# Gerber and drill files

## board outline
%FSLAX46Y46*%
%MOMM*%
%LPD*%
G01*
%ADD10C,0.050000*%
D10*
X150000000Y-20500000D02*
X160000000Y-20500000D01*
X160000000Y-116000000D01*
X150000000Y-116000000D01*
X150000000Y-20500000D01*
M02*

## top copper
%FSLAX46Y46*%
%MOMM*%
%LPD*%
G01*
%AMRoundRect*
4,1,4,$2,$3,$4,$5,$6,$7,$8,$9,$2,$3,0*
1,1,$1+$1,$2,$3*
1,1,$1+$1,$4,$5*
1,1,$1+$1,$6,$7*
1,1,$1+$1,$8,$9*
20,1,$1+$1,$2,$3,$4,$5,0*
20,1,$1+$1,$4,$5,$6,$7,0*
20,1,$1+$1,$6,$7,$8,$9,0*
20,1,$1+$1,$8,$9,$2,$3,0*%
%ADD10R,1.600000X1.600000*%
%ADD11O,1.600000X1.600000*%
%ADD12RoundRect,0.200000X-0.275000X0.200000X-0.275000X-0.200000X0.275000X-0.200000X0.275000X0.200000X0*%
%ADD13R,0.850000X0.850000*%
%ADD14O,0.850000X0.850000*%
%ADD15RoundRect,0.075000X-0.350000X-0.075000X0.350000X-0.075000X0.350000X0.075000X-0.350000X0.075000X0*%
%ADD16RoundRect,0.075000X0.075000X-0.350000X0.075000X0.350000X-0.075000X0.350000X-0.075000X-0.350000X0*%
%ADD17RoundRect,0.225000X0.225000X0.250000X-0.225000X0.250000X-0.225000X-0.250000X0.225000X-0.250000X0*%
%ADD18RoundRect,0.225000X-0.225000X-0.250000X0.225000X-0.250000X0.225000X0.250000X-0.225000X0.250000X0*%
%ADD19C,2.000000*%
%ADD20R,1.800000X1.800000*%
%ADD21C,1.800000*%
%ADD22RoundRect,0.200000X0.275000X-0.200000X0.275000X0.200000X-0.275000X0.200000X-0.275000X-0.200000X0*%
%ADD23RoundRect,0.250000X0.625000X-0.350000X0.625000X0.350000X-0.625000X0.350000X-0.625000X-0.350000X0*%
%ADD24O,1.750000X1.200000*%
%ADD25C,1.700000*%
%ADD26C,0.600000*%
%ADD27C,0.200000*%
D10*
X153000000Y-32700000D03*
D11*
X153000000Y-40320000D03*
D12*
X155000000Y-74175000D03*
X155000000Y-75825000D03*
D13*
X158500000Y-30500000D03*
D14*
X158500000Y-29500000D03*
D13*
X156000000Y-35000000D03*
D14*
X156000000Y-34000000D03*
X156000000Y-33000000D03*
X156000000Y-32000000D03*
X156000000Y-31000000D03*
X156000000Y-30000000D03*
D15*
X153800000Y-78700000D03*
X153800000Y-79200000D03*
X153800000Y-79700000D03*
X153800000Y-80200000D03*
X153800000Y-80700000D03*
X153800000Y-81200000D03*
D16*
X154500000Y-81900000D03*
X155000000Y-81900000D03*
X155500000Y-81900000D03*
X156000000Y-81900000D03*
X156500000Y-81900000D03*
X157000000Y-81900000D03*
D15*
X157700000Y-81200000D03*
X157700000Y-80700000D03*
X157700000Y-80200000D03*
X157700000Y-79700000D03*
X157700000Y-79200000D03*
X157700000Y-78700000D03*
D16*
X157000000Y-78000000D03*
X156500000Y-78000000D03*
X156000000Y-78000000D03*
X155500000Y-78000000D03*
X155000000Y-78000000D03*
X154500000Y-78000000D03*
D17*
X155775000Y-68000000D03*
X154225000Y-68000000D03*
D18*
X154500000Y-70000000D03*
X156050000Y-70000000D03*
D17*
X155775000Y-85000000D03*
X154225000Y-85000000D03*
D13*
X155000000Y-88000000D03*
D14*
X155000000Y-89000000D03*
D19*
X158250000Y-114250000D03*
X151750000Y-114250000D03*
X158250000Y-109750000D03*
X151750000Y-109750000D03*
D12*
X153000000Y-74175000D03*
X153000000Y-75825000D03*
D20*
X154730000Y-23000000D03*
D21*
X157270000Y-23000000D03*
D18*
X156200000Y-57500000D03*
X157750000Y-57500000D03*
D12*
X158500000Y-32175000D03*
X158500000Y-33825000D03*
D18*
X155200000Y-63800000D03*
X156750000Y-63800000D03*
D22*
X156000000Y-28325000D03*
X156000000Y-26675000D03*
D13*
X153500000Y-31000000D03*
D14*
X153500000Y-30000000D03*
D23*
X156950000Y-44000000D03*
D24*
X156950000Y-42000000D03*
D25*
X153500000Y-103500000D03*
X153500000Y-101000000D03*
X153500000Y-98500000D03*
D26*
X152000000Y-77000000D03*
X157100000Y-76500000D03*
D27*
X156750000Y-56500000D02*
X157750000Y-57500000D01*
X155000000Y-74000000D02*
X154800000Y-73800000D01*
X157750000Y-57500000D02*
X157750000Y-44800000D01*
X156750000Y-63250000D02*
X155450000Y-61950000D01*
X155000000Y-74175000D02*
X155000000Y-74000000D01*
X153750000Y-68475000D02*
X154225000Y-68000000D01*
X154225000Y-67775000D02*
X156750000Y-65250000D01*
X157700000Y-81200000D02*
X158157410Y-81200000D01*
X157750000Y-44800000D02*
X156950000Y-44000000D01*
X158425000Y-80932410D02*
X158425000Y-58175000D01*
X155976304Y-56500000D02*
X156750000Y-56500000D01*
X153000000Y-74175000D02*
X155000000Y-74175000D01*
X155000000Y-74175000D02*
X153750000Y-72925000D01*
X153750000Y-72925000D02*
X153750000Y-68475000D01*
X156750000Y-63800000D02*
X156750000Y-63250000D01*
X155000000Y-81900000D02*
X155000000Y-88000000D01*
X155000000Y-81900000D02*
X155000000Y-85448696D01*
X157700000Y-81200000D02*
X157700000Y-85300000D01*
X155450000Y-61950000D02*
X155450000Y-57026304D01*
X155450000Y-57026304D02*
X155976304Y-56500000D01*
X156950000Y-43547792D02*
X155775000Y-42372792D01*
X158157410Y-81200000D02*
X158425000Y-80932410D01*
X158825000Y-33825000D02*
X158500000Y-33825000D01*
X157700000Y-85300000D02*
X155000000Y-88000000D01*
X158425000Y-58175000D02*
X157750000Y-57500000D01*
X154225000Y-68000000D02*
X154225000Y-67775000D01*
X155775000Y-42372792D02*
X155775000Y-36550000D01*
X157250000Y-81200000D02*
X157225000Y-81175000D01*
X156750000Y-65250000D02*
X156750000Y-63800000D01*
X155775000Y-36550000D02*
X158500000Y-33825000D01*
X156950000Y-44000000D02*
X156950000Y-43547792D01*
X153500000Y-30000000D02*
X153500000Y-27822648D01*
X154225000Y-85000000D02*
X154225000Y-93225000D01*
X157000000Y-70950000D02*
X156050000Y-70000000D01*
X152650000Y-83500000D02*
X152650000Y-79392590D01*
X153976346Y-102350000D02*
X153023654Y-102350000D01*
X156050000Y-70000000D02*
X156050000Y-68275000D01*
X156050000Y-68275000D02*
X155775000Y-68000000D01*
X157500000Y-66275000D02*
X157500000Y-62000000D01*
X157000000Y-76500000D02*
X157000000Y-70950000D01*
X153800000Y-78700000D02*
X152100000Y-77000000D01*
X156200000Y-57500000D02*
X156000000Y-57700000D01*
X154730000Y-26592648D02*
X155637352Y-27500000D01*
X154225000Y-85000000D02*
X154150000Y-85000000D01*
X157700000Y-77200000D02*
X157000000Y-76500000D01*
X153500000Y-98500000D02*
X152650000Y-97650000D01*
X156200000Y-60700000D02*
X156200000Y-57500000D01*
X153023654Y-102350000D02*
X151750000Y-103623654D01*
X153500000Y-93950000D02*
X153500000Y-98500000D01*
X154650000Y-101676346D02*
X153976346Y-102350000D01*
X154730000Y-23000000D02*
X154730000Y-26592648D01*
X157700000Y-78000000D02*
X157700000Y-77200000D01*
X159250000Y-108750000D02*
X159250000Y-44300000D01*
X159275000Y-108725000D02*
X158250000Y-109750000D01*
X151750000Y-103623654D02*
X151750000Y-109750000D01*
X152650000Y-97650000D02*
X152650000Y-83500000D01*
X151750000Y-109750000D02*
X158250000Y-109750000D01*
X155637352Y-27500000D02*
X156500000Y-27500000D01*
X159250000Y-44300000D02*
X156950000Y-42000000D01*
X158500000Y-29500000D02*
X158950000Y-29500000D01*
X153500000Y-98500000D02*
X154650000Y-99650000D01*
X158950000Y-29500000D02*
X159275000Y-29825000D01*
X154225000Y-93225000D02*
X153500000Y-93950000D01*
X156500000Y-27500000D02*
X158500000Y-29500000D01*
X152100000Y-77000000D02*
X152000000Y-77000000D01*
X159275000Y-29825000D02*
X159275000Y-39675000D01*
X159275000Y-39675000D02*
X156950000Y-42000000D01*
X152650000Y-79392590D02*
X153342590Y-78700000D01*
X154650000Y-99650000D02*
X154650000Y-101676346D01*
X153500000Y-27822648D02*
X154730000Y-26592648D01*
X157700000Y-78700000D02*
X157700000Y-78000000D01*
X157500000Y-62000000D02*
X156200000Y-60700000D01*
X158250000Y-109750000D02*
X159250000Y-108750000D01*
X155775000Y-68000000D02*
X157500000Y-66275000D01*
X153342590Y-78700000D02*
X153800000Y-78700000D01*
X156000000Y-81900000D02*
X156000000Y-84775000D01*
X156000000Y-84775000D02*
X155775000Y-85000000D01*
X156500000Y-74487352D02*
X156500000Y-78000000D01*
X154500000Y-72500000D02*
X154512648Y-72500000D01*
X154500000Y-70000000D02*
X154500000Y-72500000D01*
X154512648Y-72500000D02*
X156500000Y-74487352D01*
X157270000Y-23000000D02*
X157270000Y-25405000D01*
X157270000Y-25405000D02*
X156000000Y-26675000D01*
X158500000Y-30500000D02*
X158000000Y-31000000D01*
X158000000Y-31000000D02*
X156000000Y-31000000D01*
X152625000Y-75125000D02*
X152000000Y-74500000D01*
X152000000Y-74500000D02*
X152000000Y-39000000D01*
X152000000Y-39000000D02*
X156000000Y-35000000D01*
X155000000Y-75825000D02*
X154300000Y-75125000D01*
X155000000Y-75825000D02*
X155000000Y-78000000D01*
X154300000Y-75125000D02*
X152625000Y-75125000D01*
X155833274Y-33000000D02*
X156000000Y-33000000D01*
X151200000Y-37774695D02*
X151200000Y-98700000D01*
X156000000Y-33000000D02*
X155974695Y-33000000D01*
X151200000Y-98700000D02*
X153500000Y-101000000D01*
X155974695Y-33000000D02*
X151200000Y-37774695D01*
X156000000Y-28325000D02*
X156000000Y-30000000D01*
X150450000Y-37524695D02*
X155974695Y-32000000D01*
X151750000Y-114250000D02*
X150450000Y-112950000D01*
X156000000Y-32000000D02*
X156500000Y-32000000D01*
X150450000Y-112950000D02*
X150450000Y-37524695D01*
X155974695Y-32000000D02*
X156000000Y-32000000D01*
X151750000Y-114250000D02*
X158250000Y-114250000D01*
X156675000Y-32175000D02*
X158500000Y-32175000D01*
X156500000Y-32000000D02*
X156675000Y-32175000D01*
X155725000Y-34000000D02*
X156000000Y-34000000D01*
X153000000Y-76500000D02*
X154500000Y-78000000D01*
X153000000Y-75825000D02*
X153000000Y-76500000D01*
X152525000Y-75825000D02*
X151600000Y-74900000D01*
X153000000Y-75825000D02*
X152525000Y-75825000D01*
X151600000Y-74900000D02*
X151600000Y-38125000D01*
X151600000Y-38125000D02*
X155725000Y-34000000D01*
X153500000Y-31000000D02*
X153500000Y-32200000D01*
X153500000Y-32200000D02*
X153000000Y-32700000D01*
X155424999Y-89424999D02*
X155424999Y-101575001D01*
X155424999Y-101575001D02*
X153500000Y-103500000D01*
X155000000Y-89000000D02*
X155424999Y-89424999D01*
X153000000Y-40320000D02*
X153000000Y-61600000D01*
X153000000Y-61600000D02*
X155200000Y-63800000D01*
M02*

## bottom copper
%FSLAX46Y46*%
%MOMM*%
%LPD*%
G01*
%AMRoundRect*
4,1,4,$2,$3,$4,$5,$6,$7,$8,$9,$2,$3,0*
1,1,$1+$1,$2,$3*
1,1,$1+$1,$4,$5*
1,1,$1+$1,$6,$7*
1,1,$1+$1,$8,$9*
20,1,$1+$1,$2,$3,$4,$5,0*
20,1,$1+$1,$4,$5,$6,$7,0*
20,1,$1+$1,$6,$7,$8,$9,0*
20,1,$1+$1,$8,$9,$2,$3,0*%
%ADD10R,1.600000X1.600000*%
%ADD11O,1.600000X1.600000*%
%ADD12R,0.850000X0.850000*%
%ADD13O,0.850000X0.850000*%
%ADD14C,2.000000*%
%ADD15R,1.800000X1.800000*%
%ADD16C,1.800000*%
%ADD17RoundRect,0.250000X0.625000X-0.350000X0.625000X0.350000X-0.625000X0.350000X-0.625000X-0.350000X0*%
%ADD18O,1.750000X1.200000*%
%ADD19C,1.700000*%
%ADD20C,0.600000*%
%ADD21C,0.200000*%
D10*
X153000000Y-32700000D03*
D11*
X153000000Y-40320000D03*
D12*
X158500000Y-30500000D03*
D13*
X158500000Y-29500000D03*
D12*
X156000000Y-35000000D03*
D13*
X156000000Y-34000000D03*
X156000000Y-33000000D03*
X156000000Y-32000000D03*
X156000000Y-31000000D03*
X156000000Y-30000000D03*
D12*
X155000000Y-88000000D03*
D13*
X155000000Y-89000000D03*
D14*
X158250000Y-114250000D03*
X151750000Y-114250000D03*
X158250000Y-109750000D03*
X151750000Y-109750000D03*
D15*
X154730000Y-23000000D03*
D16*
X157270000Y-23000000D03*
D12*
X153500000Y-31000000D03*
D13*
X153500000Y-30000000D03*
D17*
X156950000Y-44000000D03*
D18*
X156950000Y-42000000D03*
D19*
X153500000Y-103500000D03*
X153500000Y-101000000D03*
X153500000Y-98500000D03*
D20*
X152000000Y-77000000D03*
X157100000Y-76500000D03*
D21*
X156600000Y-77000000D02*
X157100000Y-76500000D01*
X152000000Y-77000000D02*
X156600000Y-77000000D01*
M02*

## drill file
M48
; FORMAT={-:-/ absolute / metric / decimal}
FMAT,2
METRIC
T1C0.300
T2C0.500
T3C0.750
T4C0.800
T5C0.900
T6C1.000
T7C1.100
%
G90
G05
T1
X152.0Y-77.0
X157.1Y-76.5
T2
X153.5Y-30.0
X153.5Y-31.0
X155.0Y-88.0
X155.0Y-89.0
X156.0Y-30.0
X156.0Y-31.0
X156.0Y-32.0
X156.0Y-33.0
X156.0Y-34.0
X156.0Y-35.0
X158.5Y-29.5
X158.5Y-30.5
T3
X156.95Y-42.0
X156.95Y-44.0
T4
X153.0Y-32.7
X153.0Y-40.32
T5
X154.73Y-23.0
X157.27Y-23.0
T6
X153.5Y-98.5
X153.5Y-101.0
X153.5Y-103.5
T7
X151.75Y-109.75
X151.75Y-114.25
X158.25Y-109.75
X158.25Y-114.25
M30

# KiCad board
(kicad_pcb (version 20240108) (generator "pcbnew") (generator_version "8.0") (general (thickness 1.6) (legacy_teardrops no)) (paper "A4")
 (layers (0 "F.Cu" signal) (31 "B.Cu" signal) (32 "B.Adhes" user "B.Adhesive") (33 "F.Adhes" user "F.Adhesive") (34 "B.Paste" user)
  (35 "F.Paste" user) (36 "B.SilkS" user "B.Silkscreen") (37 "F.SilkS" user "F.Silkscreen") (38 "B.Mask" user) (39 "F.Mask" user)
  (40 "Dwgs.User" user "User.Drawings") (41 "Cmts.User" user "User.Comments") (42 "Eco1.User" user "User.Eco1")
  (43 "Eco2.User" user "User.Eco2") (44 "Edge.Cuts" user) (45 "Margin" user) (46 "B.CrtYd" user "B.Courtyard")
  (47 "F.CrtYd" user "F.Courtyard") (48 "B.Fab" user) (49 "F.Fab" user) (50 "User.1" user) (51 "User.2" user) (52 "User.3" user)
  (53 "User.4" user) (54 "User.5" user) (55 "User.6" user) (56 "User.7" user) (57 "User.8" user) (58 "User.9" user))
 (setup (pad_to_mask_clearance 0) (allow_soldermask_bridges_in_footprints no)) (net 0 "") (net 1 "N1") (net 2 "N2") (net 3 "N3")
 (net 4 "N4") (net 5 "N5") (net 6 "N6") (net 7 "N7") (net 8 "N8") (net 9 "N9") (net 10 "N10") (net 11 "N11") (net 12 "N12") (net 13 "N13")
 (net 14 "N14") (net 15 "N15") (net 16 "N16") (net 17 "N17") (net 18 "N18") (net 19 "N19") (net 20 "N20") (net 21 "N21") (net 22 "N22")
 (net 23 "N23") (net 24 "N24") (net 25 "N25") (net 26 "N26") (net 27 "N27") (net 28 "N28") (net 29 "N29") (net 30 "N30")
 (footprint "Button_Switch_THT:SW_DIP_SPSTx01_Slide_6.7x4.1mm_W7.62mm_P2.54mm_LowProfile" (layer "F.Cu") (at 153 32.7 -90)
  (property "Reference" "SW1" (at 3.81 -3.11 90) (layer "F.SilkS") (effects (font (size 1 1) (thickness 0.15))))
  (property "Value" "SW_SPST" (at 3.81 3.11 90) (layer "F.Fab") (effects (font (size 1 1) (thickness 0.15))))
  (pad "1" thru_hole rect (at 0 0 270) (size 1.6 1.6) (drill 0.8) (layers "*.Cu" "*.Mask") (remove_unused_layers no) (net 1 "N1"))
  (pad "2" thru_hole oval (at 7.62 0 270) (size 1.6 1.6) (drill 0.8) (layers "*.Cu" "*.Mask") (remove_unused_layers no) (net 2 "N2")))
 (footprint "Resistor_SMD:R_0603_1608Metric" (layer "F.Cu") (at 155 75 -90)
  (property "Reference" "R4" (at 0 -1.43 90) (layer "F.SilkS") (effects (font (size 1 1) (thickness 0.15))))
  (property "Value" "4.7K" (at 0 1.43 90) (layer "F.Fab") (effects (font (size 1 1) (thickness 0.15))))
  (pad "1" smd roundrect (at -0.825 0 270) (size 0.8 0.95) (layers "F.Cu" "F.Paste" "F.Mask") (roundrect_rratio 0.25) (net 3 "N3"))
  (pad "2" smd roundrect (at 0.825 0 270) (size 0.8 0.95) (layers "F.Cu" "F.Paste" "F.Mask") (roundrect_rratio 0.25) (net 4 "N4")))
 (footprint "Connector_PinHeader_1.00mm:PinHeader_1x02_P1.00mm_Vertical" (layer "F.Cu") (at 158.5 30.5 180)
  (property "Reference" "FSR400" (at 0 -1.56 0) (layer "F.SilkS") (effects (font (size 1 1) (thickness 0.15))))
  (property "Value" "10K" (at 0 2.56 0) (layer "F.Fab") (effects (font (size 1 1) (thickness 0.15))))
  (pad "1" thru_hole rect (at 0 0 180) (size 0.85 0.85) (drill 0.5) (layers "*.Cu" "*.Mask") (remove_unused_layers no) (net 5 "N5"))
  (pad "2" thru_hole oval (at 0 1 180) (size 0.85 0.85) (drill 0.5) (layers "*.Cu" "*.Mask") (remove_unused_layers no) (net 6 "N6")))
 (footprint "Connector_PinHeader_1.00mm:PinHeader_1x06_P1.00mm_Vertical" (layer "F.Cu") (at 156 35 180)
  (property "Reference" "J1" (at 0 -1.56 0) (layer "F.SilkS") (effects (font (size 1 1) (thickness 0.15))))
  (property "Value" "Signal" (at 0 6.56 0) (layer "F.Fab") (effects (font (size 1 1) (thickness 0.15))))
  (pad "1" thru_hole rect (at 0 0 180) (size 0.85 0.85) (drill 0.5) (layers "*.Cu" "*.Mask") (remove_unused_layers no) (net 4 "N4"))
  (pad "2" thru_hole oval (at 0 1 180) (size 0.85 0.85) (drill 0.5) (layers "*.Cu" "*.Mask") (remove_unused_layers no) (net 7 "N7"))
  (pad "3" thru_hole oval (at 0 2 180) (size 0.85 0.85) (drill 0.5) (layers "*.Cu" "*.Mask") (remove_unused_layers no) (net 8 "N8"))
  (pad "4" thru_hole oval (at 0 3 180) (size 0.85 0.85) (drill 0.5) (layers "*.Cu" "*.Mask") (remove_unused_layers no) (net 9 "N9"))
  (pad "5" thru_hole oval (at 0 4 180) (size 0.85 0.85) (drill 0.5) (layers "*.Cu" "*.Mask") (remove_unused_layers no) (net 5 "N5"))
  (pad "6" thru_hole oval (at 0 5 180) (size 0.85 0.85) (drill 0.5) (layers "*.Cu" "*.Mask") (remove_unused_layers no) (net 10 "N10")))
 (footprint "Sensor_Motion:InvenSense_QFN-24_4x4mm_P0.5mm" (layer "F.Cu") (at 155.75 79.95)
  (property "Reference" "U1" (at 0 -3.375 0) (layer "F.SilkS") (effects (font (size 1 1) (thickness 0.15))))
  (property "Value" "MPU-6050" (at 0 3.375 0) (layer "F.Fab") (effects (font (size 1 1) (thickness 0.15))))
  (pad "1" smd roundrect (at -1.95 -1.25) (size 0.85 0.3) (layers "F.Cu" "F.Paste" "F.Mask") (roundrect_rratio 0.25) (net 6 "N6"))
  (pad "2" smd roundrect (at -1.95 -0.75) (size 0.85 0.3) (layers "F.Cu" "F.Paste" "F.Mask") (roundrect_rratio 0.25) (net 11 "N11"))
  (pad "3" smd roundrect (at -1.95 -0.25) (size 0.85 0.3) (layers "F.Cu" "F.Paste" "F.Mask") (roundrect_rratio 0.25) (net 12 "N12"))
  (pad "4" smd roundrect (at -1.95 0.25) (size 0.85 0.3) (layers "F.Cu" "F.Paste" "F.Mask") (roundrect_rratio 0.25) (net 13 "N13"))
  (pad "5" smd roundrect (at -1.95 0.75) (size 0.85 0.3) (layers "F.Cu" "F.Paste" "F.Mask") (roundrect_rratio 0.25) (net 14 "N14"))
  (pad "6" smd roundrect (at -1.95 1.25) (size 0.85 0.3) (layers "F.Cu" "F.Paste" "F.Mask") (roundrect_rratio 0.25) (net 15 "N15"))
  (pad "7" smd roundrect (at -1.25 1.95 90) (size 0.85 0.3) (layers "F.Cu" "F.Paste" "F.Mask") (roundrect_rratio 0.25) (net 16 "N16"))
  (pad "8" smd roundrect (at -0.75 1.95 90) (size 0.85 0.3) (layers "F.Cu" "F.Paste" "F.Mask") (roundrect_rratio 0.25) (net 3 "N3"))
  (pad "9" smd roundrect (at -0.25 1.95 90) (size 0.85 0.3) (layers "F.Cu" "F.Paste" "F.Mask") (roundrect_rratio 0.25) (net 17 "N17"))
  (pad "10" smd roundrect (at 0.25 1.95 90) (size 0.85 0.3) (layers "F.Cu" "F.Paste" "F.Mask") (roundrect_rratio 0.25) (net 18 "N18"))
  (pad "11" smd roundrect (at 0.75 1.95 90) (size 0.85 0.3) (layers "F.Cu" "F.Paste" "F.Mask") (roundrect_rratio 0.25) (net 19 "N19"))
  (pad "12" smd roundrect (at 1.25 1.95 90) (size 0.85 0.3) (layers "F.Cu" "F.Paste" "F.Mask") (roundrect_rratio 0.25) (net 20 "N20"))
  (pad "13" smd roundrect (at 1.95 1.25) (size 0.85 0.3) (layers "F.Cu" "F.Paste" "F.Mask") (roundrect_rratio 0.25) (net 3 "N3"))
  (pad "14" smd roundrect (at 1.95 0.75) (size 0.85 0.3) (layers "F.Cu" "F.Paste" "F.Mask") (roundrect_rratio 0.25) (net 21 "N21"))
  (pad "15" smd roundrect (at 1.95 0.25) (size 0.85 0.3) (layers "F.Cu" "F.Paste" "F.Mask") (roundrect_rratio 0.25) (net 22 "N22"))
  (pad "16" smd roundrect (at 1.95 -0.25) (size 0.85 0.3) (layers "F.Cu" "F.Paste" "F.Mask") (roundrect_rratio 0.25) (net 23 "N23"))
  (pad "17" smd roundrect (at 1.95 -0.75) (size 0.85 0.3) (layers "F.Cu" "F.Paste" "F.Mask") (roundrect_rratio 0.25) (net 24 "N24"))
  (pad "18" smd roundrect (at 1.95 -1.25) (size 0.85 0.3) (layers "F.Cu" "F.Paste" "F.Mask") (roundrect_rratio 0.25) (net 6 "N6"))
  (pad "19" smd roundrect (at 1.25 -1.95 90) (size 0.85 0.3) (layers "F.Cu" "F.Paste" "F.Mask") (roundrect_rratio 0.25) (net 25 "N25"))
  (pad "20" smd roundrect (at 0.75 -1.95 90) (size 0.85 0.3) (layers "F.Cu" "F.Paste" "F.Mask") (roundrect_rratio 0.25) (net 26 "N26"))
  (pad "21" smd roundrect (at 0.25 -1.95 90) (size 0.85 0.3) (layers "F.Cu" "F.Paste" "F.Mask") (roundrect_rratio 0.25) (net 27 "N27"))
  (pad "22" smd roundrect (at -0.25 -1.95 90) (size 0.85 0.3) (layers "F.Cu" "F.Paste" "F.Mask") (roundrect_rratio 0.25) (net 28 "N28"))
  (pad "23" smd roundrect (at -0.75 -1.95 90) (size 0.85 0.3) (layers "F.Cu" "F.Paste" "F.Mask") (roundrect_rratio 0.25) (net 4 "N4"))
  (pad "24" smd roundrect (at -1.25 -1.95 90) (size 0.85 0.3) (layers "F.Cu" "F.Paste" "F.Mask") (roundrect_rratio 0.25) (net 7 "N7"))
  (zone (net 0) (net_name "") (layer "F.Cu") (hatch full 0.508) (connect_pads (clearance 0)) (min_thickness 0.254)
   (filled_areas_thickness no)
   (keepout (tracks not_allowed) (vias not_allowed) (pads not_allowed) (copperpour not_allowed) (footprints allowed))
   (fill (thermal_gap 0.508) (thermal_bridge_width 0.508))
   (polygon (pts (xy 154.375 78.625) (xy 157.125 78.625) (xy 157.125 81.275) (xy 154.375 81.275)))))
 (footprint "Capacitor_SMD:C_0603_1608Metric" (layer "F.Cu") (at 155 68 180)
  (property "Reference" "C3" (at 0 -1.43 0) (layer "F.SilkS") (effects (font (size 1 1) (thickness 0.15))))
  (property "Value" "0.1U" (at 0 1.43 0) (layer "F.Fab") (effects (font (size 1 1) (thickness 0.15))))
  (pad "1" smd roundrect (at -0.775 0 180) (size 0.9 0.95) (layers "F.Cu" "F.Paste" "F.Mask") (roundrect_rratio 0.25) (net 6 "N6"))
  (pad "2" smd roundrect (at 0.775 0 180) (size 0.9 0.95) (layers "F.Cu" "F.Paste" "F.Mask") (roundrect_rratio 0.25) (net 3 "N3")))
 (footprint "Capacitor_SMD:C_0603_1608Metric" (layer "F.Cu") (at 155.275 70)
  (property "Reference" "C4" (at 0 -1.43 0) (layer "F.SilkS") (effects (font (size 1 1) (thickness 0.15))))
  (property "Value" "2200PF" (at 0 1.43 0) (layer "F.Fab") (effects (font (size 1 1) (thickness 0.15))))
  (pad "1" smd roundrect (at -0.775 0) (size 0.9 0.95) (layers "F.Cu" "F.Paste" "F.Mask") (roundrect_rratio 0.25) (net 26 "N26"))
  (pad "2" smd roundrect (at 0.775 0) (size 0.9 0.95) (layers "F.Cu" "F.Paste" "F.Mask") (roundrect_rratio 0.25) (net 6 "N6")))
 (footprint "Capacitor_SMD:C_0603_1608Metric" (layer "F.Cu") (at 155 85 180)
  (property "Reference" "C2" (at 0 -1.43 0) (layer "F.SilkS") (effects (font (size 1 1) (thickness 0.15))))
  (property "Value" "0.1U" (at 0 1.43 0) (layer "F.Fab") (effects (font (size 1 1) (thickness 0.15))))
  (pad "1" smd roundrect (at -0.775 0 180) (size 0.9 0.95) (layers "F.Cu" "F.Paste" "F.Mask") (roundrect_rratio 0.25) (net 18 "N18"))
  (pad "2" smd roundrect (at 0.775 0 180) (size 0.9 0.95) (layers "F.Cu" "F.Paste" "F.Mask") (roundrect_rratio 0.25) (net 6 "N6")))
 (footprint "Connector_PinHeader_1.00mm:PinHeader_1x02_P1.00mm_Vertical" (layer "F.Cu") (at 155 88)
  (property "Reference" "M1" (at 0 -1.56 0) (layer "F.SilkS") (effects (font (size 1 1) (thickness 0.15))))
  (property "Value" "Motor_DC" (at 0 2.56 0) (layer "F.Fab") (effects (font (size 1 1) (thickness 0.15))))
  (pad "1" thru_hole rect (at 0 0) (size 0.85 0.85) (drill 0.5) (layers "*.Cu" "*.Mask") (remove_unused_layers no) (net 3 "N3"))
  (pad "2" thru_hole oval (at 0 1) (size 0.85 0.85) (drill 0.5) (layers "*.Cu" "*.Mask") (remove_unused_layers no) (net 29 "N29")))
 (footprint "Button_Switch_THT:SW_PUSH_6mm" (layer "F.Cu") (at 158.25 114.25 180)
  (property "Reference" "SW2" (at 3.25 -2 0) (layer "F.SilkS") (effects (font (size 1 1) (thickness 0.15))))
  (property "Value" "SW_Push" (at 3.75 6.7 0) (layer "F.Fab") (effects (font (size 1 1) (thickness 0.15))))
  (pad "1" thru_hole circle (at 0 0 270) (size 2 2) (drill 1.1) (layers "*.Cu" "*.Mask") (remove_unused_layers no) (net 9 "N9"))
  (pad "1" thru_hole circle (at 6.5 0 270) (size 2 2) (drill 1.1) (layers "*.Cu" "*.Mask") (remove_unused_layers no) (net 9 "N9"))
  (pad "2" thru_hole circle (at 0 4.5 270) (size 2 2) (drill 1.1) (layers "*.Cu" "*.Mask") (remove_unused_layers no) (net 6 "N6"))
  (pad "2" thru_hole circle (at 6.5 4.5 270) (size 2 2) (drill 1.1) (layers "*.Cu" "*.Mask") (remove_unused_layers no) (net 6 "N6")))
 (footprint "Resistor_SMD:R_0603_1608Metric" (layer "F.Cu") (at 153 75 -90)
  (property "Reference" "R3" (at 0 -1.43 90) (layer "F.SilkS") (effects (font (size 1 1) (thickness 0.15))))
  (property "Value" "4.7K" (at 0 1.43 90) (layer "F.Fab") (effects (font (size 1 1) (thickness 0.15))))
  (pad "1" smd roundrect (at -0.825 0 270) (size 0.8 0.95) (layers "F.Cu" "F.Paste" "F.Mask") (roundrect_rratio 0.25) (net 3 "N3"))
  (pad "2" smd roundrect (at 0.825 0 270) (size 0.8 0.95) (layers "F.Cu" "F.Paste" "F.Mask") (roundrect_rratio 0.25) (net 7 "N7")))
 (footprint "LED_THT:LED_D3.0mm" (layer "F.Cu") (at 154.73 23)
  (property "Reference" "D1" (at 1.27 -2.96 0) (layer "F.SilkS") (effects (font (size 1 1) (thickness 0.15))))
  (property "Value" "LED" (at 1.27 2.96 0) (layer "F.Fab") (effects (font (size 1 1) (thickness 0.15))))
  (pad "1" thru_hole rect (at 0 0) (size 1.8 1.8) (drill 0.9) (layers "*.Cu" "*.Mask") (remove_unused_layers no) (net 6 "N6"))
  (pad "2" thru_hole circle (at 2.54 0) (size 1.8 1.8) (drill 0.9) (layers "*.Cu" "*.Mask") (remove_unused_layers no) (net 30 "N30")))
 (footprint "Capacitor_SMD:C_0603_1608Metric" (layer "F.Cu") (at 156.975 57.5)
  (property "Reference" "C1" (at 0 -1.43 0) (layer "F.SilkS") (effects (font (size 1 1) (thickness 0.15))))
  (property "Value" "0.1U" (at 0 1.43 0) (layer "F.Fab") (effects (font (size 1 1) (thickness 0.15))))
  (pad "1" smd roundrect (at -0.775 0) (size 0.9 0.95) (layers "F.Cu" "F.Paste" "F.Mask") (roundrect_rratio 0.25) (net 6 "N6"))
  (pad "2" smd roundrect (at 0.775 0) (size 0.9 0.95) (layers "F.Cu" "F.Paste" "F.Mask") (roundrect_rratio 0.25) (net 3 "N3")))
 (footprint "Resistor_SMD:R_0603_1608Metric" (layer "F.Cu") (at 158.5 33 -90)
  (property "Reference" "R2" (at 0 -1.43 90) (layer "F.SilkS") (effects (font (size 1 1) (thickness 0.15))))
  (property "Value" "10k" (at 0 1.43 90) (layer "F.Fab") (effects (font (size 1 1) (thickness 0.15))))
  (pad "1" smd roundrect (at -0.825 0 270) (size 0.8 0.95) (layers "F.Cu" "F.Paste" "F.Mask") (roundrect_rratio 0.25) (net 9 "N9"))
  (pad "2" smd roundrect (at 0.825 0 270) (size 0.8 0.95) (layers "F.Cu" "F.Paste" "F.Mask") (roundrect_rratio 0.25) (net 3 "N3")))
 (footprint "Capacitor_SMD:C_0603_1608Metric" (layer "F.Cu") (at 155.975 63.8)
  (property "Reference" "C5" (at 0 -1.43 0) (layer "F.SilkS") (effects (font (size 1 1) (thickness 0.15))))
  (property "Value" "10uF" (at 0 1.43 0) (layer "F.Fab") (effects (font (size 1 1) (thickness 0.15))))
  (pad "1" smd roundrect (at -0.775 0) (size 0.9 0.95) (layers "F.Cu" "F.Paste" "F.Mask") (roundrect_rratio 0.25) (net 2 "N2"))
  (pad "2" smd roundrect (at 0.775 0) (size 0.9 0.95) (layers "F.Cu" "F.Paste" "F.Mask") (roundrect_rratio 0.25) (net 3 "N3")))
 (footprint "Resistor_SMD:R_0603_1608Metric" (layer "F.Cu") (at 156 27.5 90)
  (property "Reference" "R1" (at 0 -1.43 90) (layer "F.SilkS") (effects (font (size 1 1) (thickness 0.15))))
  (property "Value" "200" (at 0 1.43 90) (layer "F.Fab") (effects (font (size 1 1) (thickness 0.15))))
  (pad "1" smd roundrect (at -0.825 0 90) (size 0.8 0.95) (layers "F.Cu" "F.Paste" "F.Mask") (roundrect_rratio 0.25) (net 10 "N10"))
  (pad "2" smd roundrect (at 0.825 0 90) (size 0.8 0.95) (layers "F.Cu" "F.Paste" "F.Mask") (roundrect_rratio 0.25) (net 30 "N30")))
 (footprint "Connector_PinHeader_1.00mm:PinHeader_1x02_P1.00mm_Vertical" (layer "F.Cu") (at 153.5 31 180)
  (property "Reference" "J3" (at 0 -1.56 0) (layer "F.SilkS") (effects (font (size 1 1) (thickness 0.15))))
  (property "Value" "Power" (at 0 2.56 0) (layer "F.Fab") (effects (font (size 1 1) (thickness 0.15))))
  (pad "1" thru_hole rect (at 0 0 180) (size 0.85 0.85) (drill 0.5) (layers "*.Cu" "*.Mask") (remove_unused_layers no) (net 1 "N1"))
  (pad "2" thru_hole oval (at 0 1 180) (size 0.85 0.85) (drill 0.5) (layers "*.Cu" "*.Mask") (remove_unused_layers no) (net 6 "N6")))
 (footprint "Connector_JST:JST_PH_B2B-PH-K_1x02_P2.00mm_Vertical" (layer "F.Cu") (at 156.95 44 90)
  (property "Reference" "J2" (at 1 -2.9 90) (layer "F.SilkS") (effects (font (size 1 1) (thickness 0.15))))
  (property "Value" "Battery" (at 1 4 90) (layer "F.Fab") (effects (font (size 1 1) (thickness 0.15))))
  (pad "1" thru_hole roundrect (at 0 0 90) (size 1.2 1.75) (drill 0.75) (layers "*.Cu" "*.Mask") (remove_unused_layers no)
   (roundrect_rratio 0.208333) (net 3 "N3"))
  (pad "2" thru_hole oval (at 2 0 90) (size 1.2 1.75) (drill 0.75) (layers "*.Cu" "*.Mask") (remove_unused_layers no) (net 6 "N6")))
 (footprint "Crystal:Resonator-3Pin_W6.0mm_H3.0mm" (layer "F.Cu") (at 153.5 103.5 90)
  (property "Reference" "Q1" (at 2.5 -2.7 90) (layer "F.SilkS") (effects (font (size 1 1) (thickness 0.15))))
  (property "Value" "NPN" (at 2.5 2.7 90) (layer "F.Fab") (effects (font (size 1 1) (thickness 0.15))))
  (pad "1" thru_hole circle (at 0 0 90) (size 1.7 1.7) (drill 1) (layers "*.Cu" "*.Mask") (remove_unused_layers no) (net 29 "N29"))
  (pad "2" thru_hole circle (at 2.5 0 90) (size 1.7 1.7) (drill 1) (layers "*.Cu" "*.Mask") (remove_unused_layers no) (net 8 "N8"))
  (pad "3" thru_hole circle (at 5 0 90) (size 1.7 1.7) (drill 1) (layers "*.Cu" "*.Mask") (remove_unused_layers no) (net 6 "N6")))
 (gr_rect (start 150 20.5) (end 160 116) (stroke (width 0.05) (type default)) (fill none) (layer "Edge.Cuts"))
 (segment (start 156.75 56.5) (end 157.75 57.5) (width 0.2) (layer "F.Cu") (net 3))
 (segment (start 155 74) (end 154.8 73.8) (width 0.2) (layer "F.Cu") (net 3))
 (segment (start 157.75 57.5) (end 157.75 44.8) (width 0.2) (layer "F.Cu") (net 3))
 (segment (start 156.75 63.25) (end 155.45 61.95) (width 0.2) (layer "F.Cu") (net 3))
 (segment (start 155 74.175) (end 155 74) (width 0.2) (layer "F.Cu") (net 3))
 (segment (start 153.75 68.475) (end 154.225 68) (width 0.2) (layer "F.Cu") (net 3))
 (segment (start 154.225 67.775) (end 156.75 65.25) (width 0.2) (layer "F.Cu") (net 3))
 (segment (start 157.7 81.2) (end 158.15741 81.2) (width 0.2) (layer "F.Cu") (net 3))
 (segment (start 157.75 44.8) (end 156.95 44) (width 0.2) (layer "F.Cu") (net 3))
 (segment (start 158.425 80.93241) (end 158.425 58.175) (width 0.2) (layer "F.Cu") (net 3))
 (segment (start 155.976304 56.5) (end 156.75 56.5) (width 0.2) (layer "F.Cu") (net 3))
 (segment (start 153 74.175) (end 155 74.175) (width 0.2) (layer "F.Cu") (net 3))
 (segment (start 155 74.175) (end 153.75 72.925) (width 0.2) (layer "F.Cu") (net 3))
 (segment (start 153.75 72.925) (end 153.75 68.475) (width 0.2) (layer "F.Cu") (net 3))
 (segment (start 156.75 63.8) (end 156.75 63.25) (width 0.2) (layer "F.Cu") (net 3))
 (segment (start 155 81.9) (end 155 88) (width 0.2) (layer "F.Cu") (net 3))
 (segment (start 155 81.9) (end 155 85.448696) (width 0.2) (layer "F.Cu") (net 3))
 (segment (start 157.7 81.2) (end 157.7 85.3) (width 0.2) (layer "F.Cu") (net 3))
 (segment (start 155.45 61.95) (end 155.45 57.026304) (width 0.2) (layer "F.Cu") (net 3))
 (segment (start 155.45 57.026304) (end 155.976304 56.5) (width 0.2) (layer "F.Cu") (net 3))
 (segment (start 156.95 43.547792) (end 155.775 42.372792) (width 0.2) (layer "F.Cu") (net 3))
 (segment (start 158.15741 81.2) (end 158.425 80.93241) (width 0.2) (layer "F.Cu") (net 3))
 (segment (start 158.825 33.825) (end 158.5 33.825) (width 0.2) (layer "F.Cu") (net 3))
 (segment (start 157.7 85.3) (end 155 88) (width 0.2) (layer "F.Cu") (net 3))
 (segment (start 158.425 58.175) (end 157.75 57.5) (width 0.2) (layer "F.Cu") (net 3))
 (segment (start 154.225 68) (end 154.225 67.775) (width 0.2) (layer "F.Cu") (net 3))
 (segment (start 155.775 42.372792) (end 155.775 36.55) (width 0.2) (layer "F.Cu") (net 3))
 (segment (start 157.25 81.2) (end 157.225 81.175) (width 0.2) (layer "F.Cu") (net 3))
 (segment (start 156.75 65.25) (end 156.75 63.8) (width 0.2) (layer "F.Cu") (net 3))
 (segment (start 155.775 36.55) (end 158.5 33.825) (width 0.2) (layer "F.Cu") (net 3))
 (segment (start 156.95 44) (end 156.95 43.547792) (width 0.2) (layer "F.Cu") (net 3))
 (segment (start 153.5 30) (end 153.5 27.822648) (width 0.2) (layer "F.Cu") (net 6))
 (segment (start 154.225 85) (end 154.225 93.225) (width 0.2) (layer "F.Cu") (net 6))
 (segment (start 157 70.95) (end 156.05 70) (width 0.2) (layer "F.Cu") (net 6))
 (segment (start 152.65 83.5) (end 152.65 79.39259) (width 0.2) (layer "F.Cu") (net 6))
 (segment (start 153.976346 102.35) (end 153.023654 102.35) (width 0.2) (layer "F.Cu") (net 6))
 (segment (start 156.05 70) (end 156.05 68.275) (width 0.2) (layer "F.Cu") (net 6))
 (segment (start 156.05 68.275) (end 155.775 68) (width 0.2) (layer "F.Cu") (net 6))
 (segment (start 157.5 66.275) (end 157.5 62) (width 0.2) (layer "F.Cu") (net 6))
 (segment (start 157 76.5) (end 157 70.95) (width 0.2) (layer "F.Cu") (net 6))
 (segment (start 153.8 78.7) (end 152.1 77) (width 0.2) (layer "F.Cu") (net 6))
 (segment (start 156.2 57.5) (end 156 57.7) (width 0.2) (layer "F.Cu") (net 6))
 (segment (start 154.73 26.592648) (end 155.637352 27.5) (width 0.2) (layer "F.Cu") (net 6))
 (segment (start 154.225 85) (end 154.15 85) (width 0.2) (layer "F.Cu") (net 6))
 (segment (start 157.7 77.2) (end 157 76.5) (width 0.2) (layer "F.Cu") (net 6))
 (segment (start 153.5 98.5) (end 152.65 97.65) (width 0.2) (layer "F.Cu") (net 6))
 (segment (start 156.2 60.7) (end 156.2 57.5) (width 0.2) (layer "F.Cu") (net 6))
 (segment (start 153.023654 102.35) (end 151.75 103.623654) (width 0.2) (layer "F.Cu") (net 6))
 (segment (start 153.5 93.95) (end 153.5 98.5) (width 0.2) (layer "F.Cu") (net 6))
 (segment (start 154.65 101.676346) (end 153.976346 102.35) (width 0.2) (layer "F.Cu") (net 6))
 (segment (start 154.73 23) (end 154.73 26.592648) (width 0.2) (layer "F.Cu") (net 6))
 (segment (start 157.7 78) (end 157.7 77.2) (width 0.2) (layer "F.Cu") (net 6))
 (segment (start 159.25 108.75) (end 159.25 44.3) (width 0.2) (layer "F.Cu") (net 6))
 (segment (start 159.275 108.725) (end 158.25 109.75) (width 0.2) (layer "F.Cu") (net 6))
 (segment (start 151.75 103.623654) (end 151.75 109.75) (width 0.2) (layer "F.Cu") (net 6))
 (segment (start 152.65 97.65) (end 152.65 83.5) (width 0.2) (layer "F.Cu") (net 6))
 (segment (start 151.75 109.75) (end 158.25 109.75) (width 0.2) (layer "F.Cu") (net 6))
 (segment (start 155.637352 27.5) (end 156.5 27.5) (width 0.2) (layer "F.Cu") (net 6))
 (segment (start 159.25 44.3) (end 156.95 42) (width 0.2) (layer "F.Cu") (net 6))
 (segment (start 158.5 29.5) (end 158.95 29.5) (width 0.2) (layer "F.Cu") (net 6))
 (segment (start 153.5 98.5) (end 154.65 99.65) (width 0.2) (layer "F.Cu") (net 6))
 (segment (start 158.95 29.5) (end 159.275 29.825) (width 0.2) (layer "F.Cu") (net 6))
 (segment (start 154.225 93.225) (end 153.5 93.95) (width 0.2) (layer "F.Cu") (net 6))
 (segment (start 156.5 27.5) (end 158.5 29.5) (width 0.2) (layer "F.Cu") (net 6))
 (segment (start 152.1 77) (end 152 77) (width 0.2) (layer "F.Cu") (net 6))
 (segment (start 159.275 29.825) (end 159.275 39.675) (width 0.2) (layer "F.Cu") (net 6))
 (segment (start 159.275 39.675) (end 156.95 42) (width 0.2) (layer "F.Cu") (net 6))
 (segment (start 152.65 79.39259) (end 153.34259 78.7) (width 0.2) (layer "F.Cu") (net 6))
 (segment (start 154.65 99.65) (end 154.65 101.676346) (width 0.2) (layer "F.Cu") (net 6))
 (segment (start 153.5 27.822648) (end 154.73 26.592648) (width 0.2) (layer "F.Cu") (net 6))
 (segment (start 157.7 78.7) (end 157.7 78) (width 0.2) (layer "F.Cu") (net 6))
 (segment (start 157.5 62) (end 156.2 60.7) (width 0.2) (layer "F.Cu") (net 6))
 (segment (start 158.25 109.75) (end 159.25 108.75) (width 0.2) (layer "F.Cu") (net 6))
 (segment (start 155.775 68) (end 157.5 66.275) (width 0.2) (layer "F.Cu") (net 6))
 (segment (start 153.34259 78.7) (end 153.8 78.7) (width 0.2) (layer "F.Cu") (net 6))
 (via (at 152 77) (size 0.6) (drill 0.3) (layers "F.Cu" "B.Cu") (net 6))
 (via (at 157.1 76.5) (size 0.6) (drill 0.3) (layers "F.Cu" "B.Cu") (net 6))
 (segment (start 156.6 77) (end 157.1 76.5) (width 0.2) (layer "B.Cu") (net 6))
 (segment (start 152 77) (end 156.6 77) (width 0.2) (layer "B.Cu") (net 6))
 (segment (start 156 81.9) (end 156 84.775) (width 0.2) (layer "F.Cu") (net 18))
 (segment (start 156 84.775) (end 155.775 85) (width 0.2) (layer "F.Cu") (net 18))
 (segment (start 156.5 74.487352) (end 156.5 78) (width 0.2) (layer "F.Cu") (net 26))
 (segment (start 154.5 72.5) (end 154.512648 72.5) (width 0.2) (layer "F.Cu") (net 26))
 (segment (start 154.5 70) (end 154.5 72.5) (width 0.2) (layer "F.Cu") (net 26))
 (segment (start 154.512648 72.5) (end 156.5 74.487352) (width 0.2) (layer "F.Cu") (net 26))
 (segment (start 157.27 23) (end 157.27 25.405) (width 0.2) (layer "F.Cu") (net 30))
 (segment (start 157.27 25.405) (end 156 26.675) (width 0.2) (layer "F.Cu") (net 30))
 (segment (start 158.5 30.5) (end 158 31) (width 0.2) (layer "F.Cu") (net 5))
 (segment (start 158 31) (end 156 31) (width 0.2) (layer "F.Cu") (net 5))
 (segment (start 152.625 75.125) (end 152 74.5) (width 0.2) (layer "F.Cu") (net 4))
 (segment (start 152 74.5) (end 152 39) (width 0.2) (layer "F.Cu") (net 4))
 (segment (start 152 39) (end 156 35) (width 0.2) (layer "F.Cu") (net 4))
 (segment (start 155 75.825) (end 154.3 75.125) (width 0.2) (layer "F.Cu") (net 4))
 (segment (start 155 75.825) (end 155 78) (width 0.2) (layer "F.Cu") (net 4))
 (segment (start 154.3 75.125) (end 152.625 75.125) (width 0.2) (layer "F.Cu") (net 4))
 (segment (start 155.833274 33) (end 156 33) (width 0.2) (layer "F.Cu") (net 8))
 (segment (start 151.2 37.774695) (end 151.2 98.7) (width 0.2) (layer "F.Cu") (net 8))
 (segment (start 156 33) (end 155.974695 33) (width 0.2) (layer "F.Cu") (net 8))
 (segment (start 151.2 98.7) (end 153.5 101) (width 0.2) (layer "F.Cu") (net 8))
 (segment (start 155.974695 33) (end 151.2 37.774695) (width 0.2) (layer "F.Cu") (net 8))
 (segment (start 156 28.325) (end 156 30) (width 0.2) (layer "F.Cu") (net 10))
 (segment (start 150.45 37.524695) (end 155.974695 32) (width 0.2) (layer "F.Cu") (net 9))
 (segment (start 151.75 114.25) (end 150.45 112.95) (width 0.2) (layer "F.Cu") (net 9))
 (segment (start 156 32) (end 156.5 32) (width 0.2) (layer "F.Cu") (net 9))
 (segment (start 150.45 112.95) (end 150.45 37.524695) (width 0.2) (layer "F.Cu") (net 9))
 (segment (start 155.974695 32) (end 156 32) (width 0.2) (layer "F.Cu") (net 9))
 (segment (start 151.75 114.25) (end 158.25 114.25) (width 0.2) (layer "F.Cu") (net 9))
 (segment (start 156.675 32.175) (end 158.5 32.175) (width 0.2) (layer "F.Cu") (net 9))
 (segment (start 156.5 32) (end 156.675 32.175) (width 0.2) (layer "F.Cu") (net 9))
 (segment (start 155.725 34) (end 156 34) (width 0.2) (layer "F.Cu") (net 7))
 (segment (start 153 76.5) (end 154.5 78) (width 0.2) (layer "F.Cu") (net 7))
 (segment (start 153 75.825) (end 153 76.5) (width 0.2) (layer "F.Cu") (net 7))
 (segment (start 152.525 75.825) (end 151.6 74.9) (width 0.2) (layer "F.Cu") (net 7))
 (segment (start 153 75.825) (end 152.525 75.825) (width 0.2) (layer "F.Cu") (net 7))
 (segment (start 151.6 74.9) (end 151.6 38.125) (width 0.2) (layer "F.Cu") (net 7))
 (segment (start 151.6 38.125) (end 155.725 34) (width 0.2) (layer "F.Cu") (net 7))
 (segment (start 153.5 31) (end 153.5 32.2) (width 0.2) (layer "F.Cu") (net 1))
 (segment (start 153.5 32.2) (end 153 32.7) (width 0.2) (layer "F.Cu") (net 1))
 (segment (start 155.424999 89.424999) (end 155.424999 101.575001) (width 0.2) (layer "F.Cu") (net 29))
 (segment (start 155.424999 101.575001) (end 153.5 103.5) (width 0.2) (layer "F.Cu") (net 29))
 (segment (start 155 89) (end 155.424999 89.424999) (width 0.2) (layer "F.Cu") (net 29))
 (segment (start 153 40.32) (end 153 61.6) (width 0.2) (layer "F.Cu") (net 2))
 (segment (start 153 61.6) (end 155.2 63.8) (width 0.2) (layer "F.Cu") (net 2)))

